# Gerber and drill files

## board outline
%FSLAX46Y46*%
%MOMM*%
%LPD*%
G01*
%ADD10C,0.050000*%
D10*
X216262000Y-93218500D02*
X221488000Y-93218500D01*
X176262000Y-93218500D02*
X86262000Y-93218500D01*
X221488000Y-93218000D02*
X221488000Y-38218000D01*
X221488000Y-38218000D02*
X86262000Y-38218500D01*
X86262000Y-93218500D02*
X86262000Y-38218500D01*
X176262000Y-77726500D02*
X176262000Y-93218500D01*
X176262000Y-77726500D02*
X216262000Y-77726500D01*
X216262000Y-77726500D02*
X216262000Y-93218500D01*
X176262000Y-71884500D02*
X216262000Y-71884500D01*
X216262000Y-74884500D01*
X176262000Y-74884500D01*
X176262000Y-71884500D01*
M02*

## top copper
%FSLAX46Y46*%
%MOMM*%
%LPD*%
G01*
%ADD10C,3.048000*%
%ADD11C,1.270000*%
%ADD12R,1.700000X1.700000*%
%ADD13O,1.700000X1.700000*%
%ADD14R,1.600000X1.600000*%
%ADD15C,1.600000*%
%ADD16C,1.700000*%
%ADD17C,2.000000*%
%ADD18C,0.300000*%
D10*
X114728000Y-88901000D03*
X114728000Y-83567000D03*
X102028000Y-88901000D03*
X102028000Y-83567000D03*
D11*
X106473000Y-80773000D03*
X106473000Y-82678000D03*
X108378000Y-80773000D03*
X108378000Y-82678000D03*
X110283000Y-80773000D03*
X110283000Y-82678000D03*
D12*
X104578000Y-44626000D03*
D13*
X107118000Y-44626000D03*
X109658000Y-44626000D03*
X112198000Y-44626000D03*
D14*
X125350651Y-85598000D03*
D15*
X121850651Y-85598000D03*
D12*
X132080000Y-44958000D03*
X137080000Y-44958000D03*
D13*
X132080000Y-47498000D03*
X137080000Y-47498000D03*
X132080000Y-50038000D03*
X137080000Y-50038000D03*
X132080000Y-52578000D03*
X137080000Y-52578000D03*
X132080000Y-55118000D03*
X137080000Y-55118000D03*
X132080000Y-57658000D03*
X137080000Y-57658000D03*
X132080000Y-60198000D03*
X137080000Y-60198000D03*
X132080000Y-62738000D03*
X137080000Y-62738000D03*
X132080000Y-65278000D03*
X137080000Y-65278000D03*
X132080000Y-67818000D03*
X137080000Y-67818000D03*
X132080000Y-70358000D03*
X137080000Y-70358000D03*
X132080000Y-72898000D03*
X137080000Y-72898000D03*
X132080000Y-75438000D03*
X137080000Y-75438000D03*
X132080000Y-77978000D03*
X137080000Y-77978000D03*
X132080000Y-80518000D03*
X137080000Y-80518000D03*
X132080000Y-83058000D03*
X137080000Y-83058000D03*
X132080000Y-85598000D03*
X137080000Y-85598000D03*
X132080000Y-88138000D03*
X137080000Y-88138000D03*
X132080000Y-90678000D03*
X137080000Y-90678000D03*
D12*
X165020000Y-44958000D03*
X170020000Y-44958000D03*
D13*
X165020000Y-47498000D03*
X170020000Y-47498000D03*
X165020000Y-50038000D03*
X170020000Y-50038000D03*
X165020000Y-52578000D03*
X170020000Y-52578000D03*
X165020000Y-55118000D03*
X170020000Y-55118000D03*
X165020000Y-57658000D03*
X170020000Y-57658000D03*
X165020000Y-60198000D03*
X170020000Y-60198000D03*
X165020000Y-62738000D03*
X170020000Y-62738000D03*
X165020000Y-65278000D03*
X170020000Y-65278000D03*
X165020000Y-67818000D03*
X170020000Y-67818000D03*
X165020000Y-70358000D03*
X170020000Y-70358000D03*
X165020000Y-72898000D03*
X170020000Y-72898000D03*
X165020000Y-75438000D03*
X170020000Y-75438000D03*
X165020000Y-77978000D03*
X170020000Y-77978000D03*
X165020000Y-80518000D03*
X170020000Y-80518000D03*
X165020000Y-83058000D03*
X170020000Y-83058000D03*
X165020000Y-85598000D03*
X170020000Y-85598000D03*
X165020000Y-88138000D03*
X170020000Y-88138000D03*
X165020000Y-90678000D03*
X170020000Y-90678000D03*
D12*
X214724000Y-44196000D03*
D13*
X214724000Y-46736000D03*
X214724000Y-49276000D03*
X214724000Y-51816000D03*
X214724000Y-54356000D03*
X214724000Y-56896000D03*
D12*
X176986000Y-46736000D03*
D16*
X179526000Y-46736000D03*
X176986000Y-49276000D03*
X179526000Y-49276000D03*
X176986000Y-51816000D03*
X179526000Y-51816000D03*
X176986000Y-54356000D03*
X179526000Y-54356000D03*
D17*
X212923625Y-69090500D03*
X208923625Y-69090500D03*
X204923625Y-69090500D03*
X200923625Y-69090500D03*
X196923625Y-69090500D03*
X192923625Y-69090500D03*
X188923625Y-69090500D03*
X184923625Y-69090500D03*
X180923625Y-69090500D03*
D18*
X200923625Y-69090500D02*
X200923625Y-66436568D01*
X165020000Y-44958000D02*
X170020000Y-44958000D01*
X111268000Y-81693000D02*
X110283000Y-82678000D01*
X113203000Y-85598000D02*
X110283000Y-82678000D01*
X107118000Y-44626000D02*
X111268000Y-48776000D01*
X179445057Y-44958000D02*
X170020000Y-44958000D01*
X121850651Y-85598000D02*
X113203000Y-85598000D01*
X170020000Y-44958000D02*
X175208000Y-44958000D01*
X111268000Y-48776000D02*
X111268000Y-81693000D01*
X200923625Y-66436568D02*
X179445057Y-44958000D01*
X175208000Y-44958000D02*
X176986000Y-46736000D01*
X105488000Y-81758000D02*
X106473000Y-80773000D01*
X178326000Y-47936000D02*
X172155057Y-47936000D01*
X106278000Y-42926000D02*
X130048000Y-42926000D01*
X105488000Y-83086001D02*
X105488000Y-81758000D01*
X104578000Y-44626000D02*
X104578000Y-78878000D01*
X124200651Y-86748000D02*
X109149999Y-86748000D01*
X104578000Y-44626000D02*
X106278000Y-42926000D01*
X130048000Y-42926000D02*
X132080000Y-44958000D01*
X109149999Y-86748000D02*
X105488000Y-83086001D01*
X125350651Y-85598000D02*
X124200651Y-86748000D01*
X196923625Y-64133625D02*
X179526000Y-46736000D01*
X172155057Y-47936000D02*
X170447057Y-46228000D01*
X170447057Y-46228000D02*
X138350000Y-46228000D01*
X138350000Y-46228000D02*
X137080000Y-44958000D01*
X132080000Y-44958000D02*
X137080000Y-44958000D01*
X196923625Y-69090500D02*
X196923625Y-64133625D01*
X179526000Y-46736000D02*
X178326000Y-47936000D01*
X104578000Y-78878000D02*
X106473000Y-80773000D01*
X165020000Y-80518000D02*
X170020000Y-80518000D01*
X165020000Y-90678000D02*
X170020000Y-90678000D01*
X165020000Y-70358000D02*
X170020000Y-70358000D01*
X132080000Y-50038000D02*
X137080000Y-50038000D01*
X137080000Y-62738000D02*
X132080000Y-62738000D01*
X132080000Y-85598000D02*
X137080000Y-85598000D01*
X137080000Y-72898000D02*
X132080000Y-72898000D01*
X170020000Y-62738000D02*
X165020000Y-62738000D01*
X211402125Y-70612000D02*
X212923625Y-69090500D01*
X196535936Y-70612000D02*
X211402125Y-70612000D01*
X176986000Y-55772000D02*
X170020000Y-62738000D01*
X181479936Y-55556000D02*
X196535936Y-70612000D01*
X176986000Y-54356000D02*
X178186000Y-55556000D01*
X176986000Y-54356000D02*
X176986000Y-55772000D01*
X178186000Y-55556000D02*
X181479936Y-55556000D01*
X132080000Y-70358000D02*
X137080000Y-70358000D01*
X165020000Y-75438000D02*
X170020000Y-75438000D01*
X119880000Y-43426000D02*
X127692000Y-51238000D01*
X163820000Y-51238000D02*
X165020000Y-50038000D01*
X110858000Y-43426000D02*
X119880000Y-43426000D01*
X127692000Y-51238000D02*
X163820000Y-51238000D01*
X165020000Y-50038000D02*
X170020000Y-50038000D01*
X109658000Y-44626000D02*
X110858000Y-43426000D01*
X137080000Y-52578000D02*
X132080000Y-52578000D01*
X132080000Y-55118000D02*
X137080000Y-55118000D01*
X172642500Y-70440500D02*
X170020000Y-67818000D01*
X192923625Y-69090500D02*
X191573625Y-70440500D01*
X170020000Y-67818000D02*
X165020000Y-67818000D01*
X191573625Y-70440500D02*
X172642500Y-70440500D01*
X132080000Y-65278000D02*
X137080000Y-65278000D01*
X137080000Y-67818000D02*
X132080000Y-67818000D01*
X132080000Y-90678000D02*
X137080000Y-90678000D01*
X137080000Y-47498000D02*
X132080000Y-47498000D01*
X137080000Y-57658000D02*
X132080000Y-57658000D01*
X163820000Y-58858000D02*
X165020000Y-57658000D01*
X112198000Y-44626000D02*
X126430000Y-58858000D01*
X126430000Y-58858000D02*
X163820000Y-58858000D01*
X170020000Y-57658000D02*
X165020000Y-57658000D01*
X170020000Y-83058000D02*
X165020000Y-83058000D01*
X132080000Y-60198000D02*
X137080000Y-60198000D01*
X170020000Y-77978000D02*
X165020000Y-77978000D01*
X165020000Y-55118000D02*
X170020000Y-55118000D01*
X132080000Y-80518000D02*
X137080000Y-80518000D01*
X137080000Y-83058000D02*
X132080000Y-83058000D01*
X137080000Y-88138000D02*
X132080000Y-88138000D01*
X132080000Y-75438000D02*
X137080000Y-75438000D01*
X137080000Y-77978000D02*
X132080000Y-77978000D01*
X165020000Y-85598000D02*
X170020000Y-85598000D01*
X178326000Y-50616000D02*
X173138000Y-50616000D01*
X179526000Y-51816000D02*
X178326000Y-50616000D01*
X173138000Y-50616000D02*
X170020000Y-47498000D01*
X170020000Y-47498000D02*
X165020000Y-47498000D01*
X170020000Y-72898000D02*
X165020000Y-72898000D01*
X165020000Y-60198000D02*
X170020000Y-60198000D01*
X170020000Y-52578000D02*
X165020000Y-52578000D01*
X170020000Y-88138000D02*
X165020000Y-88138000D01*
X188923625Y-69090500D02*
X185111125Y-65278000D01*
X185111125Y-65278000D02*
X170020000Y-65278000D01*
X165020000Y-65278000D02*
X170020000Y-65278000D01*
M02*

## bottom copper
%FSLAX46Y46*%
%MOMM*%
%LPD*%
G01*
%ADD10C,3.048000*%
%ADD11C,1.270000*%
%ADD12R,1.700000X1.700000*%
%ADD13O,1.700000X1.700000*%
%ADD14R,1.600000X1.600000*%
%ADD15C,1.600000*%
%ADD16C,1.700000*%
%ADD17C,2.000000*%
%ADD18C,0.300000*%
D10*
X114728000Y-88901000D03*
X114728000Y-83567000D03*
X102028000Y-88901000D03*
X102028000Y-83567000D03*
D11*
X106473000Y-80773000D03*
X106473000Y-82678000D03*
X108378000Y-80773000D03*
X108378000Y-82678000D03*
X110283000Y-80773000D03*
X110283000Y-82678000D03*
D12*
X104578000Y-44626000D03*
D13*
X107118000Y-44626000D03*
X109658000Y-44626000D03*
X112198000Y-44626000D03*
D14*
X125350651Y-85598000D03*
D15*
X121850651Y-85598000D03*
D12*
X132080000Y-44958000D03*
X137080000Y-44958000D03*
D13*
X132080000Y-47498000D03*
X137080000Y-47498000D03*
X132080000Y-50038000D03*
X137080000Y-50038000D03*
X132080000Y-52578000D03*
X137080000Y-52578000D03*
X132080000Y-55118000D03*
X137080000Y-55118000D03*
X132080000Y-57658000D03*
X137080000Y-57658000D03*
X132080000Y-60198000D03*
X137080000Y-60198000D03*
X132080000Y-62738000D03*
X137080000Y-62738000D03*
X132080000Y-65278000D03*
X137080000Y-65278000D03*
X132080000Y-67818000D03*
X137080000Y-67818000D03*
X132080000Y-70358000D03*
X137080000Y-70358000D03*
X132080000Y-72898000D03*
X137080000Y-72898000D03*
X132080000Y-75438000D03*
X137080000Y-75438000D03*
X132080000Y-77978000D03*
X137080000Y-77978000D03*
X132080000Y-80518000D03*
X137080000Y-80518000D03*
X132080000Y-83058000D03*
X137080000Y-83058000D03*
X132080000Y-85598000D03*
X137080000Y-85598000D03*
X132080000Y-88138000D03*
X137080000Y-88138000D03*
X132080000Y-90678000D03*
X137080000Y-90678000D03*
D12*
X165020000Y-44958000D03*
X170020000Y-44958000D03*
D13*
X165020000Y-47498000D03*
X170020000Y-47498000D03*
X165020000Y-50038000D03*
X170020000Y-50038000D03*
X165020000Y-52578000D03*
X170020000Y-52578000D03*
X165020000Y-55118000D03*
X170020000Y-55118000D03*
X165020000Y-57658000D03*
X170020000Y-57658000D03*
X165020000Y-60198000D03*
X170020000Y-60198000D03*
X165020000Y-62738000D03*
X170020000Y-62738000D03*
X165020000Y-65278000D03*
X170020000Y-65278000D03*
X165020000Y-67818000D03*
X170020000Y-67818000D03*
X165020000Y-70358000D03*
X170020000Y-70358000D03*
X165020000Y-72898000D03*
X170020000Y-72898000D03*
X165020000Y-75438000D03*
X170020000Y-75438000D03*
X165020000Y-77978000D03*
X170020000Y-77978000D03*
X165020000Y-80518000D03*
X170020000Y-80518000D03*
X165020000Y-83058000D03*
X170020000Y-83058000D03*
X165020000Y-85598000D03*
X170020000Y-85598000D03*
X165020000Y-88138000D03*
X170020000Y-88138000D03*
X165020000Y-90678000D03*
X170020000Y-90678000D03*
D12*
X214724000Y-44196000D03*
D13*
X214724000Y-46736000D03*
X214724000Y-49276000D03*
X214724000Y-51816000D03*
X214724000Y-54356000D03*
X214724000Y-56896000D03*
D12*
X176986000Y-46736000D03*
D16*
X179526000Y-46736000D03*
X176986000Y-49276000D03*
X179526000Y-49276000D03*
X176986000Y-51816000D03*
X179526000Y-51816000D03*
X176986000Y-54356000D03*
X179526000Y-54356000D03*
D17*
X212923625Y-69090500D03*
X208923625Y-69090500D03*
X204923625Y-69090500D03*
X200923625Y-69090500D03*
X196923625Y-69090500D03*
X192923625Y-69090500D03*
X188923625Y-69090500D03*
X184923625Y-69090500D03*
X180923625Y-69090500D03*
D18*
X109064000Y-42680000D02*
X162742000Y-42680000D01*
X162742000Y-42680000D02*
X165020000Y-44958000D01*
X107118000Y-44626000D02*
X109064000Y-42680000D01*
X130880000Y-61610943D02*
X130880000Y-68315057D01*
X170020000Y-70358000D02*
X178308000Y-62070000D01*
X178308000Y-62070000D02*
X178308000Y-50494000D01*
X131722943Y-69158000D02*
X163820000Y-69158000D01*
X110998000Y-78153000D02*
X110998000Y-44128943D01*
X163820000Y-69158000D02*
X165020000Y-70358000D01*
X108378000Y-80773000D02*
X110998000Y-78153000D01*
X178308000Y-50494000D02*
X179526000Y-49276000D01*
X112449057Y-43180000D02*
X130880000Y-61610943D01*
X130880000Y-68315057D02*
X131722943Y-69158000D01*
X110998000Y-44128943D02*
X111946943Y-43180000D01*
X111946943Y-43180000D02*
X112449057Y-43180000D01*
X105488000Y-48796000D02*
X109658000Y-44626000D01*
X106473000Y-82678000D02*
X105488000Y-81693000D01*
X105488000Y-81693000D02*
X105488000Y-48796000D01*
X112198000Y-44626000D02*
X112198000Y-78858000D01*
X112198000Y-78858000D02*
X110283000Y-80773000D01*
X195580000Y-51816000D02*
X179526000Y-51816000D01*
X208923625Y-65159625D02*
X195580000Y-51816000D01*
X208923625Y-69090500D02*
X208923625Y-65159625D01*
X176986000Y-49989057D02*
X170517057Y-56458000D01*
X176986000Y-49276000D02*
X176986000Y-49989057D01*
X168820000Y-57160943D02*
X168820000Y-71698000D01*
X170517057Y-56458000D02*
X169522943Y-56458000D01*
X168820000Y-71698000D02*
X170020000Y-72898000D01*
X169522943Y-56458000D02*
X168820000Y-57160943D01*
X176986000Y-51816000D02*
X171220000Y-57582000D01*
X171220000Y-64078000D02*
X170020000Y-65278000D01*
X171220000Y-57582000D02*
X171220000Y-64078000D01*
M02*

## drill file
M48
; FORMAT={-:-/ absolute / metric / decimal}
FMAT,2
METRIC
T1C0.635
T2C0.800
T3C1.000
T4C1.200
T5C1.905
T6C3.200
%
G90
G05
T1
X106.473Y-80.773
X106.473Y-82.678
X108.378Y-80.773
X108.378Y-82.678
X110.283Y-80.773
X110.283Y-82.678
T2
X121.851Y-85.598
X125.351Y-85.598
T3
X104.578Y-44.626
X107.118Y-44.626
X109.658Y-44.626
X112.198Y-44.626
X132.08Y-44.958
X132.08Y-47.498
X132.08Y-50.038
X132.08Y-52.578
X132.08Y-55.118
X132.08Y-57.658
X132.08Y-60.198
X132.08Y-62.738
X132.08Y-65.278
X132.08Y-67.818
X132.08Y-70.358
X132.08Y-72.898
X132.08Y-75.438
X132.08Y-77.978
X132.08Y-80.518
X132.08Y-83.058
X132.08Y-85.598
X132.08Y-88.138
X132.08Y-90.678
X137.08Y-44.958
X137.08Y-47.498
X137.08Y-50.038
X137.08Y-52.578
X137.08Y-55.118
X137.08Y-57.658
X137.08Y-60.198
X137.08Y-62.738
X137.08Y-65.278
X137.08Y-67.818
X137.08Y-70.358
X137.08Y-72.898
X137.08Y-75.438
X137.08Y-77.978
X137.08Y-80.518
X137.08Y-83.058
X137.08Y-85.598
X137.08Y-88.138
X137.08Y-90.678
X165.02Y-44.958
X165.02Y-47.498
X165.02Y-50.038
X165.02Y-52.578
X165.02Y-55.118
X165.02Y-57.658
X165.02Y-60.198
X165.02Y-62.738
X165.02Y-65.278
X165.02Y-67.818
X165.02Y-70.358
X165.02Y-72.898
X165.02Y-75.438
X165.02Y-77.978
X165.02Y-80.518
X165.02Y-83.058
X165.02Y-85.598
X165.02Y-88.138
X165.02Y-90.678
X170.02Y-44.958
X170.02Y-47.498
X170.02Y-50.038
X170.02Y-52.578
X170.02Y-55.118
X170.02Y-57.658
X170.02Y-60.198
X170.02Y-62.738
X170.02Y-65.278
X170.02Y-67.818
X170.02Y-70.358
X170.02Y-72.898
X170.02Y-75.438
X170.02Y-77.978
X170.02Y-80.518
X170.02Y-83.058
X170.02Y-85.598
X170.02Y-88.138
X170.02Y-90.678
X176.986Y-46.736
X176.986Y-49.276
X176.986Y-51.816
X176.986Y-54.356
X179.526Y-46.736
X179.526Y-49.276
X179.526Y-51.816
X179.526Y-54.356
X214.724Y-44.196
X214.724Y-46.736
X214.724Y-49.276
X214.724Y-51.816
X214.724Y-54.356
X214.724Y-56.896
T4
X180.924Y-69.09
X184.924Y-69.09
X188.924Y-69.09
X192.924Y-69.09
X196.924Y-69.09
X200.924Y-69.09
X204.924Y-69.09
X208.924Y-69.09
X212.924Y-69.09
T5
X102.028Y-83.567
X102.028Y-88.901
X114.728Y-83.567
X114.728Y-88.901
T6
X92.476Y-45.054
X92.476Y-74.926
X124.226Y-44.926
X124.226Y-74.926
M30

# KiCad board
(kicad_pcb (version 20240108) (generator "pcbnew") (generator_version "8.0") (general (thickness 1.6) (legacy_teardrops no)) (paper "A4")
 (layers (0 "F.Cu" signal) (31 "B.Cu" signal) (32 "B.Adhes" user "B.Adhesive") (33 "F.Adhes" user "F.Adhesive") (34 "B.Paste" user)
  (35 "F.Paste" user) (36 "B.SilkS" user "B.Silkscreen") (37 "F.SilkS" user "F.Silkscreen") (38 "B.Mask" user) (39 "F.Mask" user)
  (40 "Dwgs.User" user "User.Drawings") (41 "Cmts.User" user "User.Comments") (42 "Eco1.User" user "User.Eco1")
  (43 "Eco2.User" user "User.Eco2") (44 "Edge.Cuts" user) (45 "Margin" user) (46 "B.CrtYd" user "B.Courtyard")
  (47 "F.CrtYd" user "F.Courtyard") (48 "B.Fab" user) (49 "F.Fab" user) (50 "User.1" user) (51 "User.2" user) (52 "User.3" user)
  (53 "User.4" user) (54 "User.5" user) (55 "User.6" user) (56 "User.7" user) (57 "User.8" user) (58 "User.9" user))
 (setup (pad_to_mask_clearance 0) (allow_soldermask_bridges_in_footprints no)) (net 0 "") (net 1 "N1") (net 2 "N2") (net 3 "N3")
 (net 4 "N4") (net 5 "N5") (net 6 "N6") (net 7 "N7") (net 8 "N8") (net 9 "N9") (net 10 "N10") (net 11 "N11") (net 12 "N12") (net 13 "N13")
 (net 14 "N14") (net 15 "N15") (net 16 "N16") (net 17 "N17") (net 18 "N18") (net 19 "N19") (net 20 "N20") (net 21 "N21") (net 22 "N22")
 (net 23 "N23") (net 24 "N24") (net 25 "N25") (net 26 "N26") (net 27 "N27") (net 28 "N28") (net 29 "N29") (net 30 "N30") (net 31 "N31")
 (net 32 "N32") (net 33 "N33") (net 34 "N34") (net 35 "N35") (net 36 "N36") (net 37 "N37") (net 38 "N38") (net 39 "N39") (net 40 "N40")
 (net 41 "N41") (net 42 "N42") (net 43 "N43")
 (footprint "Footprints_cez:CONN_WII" (layer "F.Cu") (at 108.378 86.361 180)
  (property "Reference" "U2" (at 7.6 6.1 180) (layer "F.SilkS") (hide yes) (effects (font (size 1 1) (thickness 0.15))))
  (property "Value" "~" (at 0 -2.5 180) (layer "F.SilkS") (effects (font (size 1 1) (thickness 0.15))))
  (pad "" thru_hole circle (at -6.35 -2.54 180) (size 3.048 3.048) (drill 1.905) (layers "*.Cu" "*.Mask") (remove_unused_layers no))
  (pad "" thru_hole circle (at -6.35 2.794 180) (size 3.048 3.048) (drill 1.905) (layers "*.Cu" "*.Mask") (remove_unused_layers no))
  (pad "" thru_hole circle (at 6.35 -2.54 180) (size 3.048 3.048) (drill 1.905) (layers "*.Cu" "*.Mask") (remove_unused_layers no))
  (pad "" thru_hole circle (at 6.35 2.794 180) (size 3.048 3.048) (drill 1.905) (layers "*.Cu" "*.Mask") (remove_unused_layers no))
  (pad "1" thru_hole circle (at 1.905 5.588 180) (size 1.27 1.27) (drill 0.635) (layers "*.Cu" "*.Mask") (remove_unused_layers no)
   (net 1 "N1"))
  (pad "2" thru_hole circle (at 1.905 3.683 180) (size 1.27 1.27) (drill 0.635) (layers "*.Cu" "*.Mask") (remove_unused_layers no)
   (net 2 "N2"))
  (pad "3" thru_hole circle (at 0 5.588 180) (size 1.27 1.27) (drill 0.635) (layers "*.Cu" "*.Mask") (remove_unused_layers no) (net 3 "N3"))
  (pad "4" thru_hole circle (at 0 3.683 180) (size 1.27 1.27) (drill 0.635) (layers "*.Cu" "*.Mask") (remove_unused_layers no) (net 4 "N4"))
  (pad "5" thru_hole circle (at -1.905 5.588 180) (size 1.27 1.27) (drill 0.635) (layers "*.Cu" "*.Mask") (remove_unused_layers no)
   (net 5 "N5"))
  (pad "6" thru_hole circle (at -1.905 3.683 180) (size 1.27 1.27) (drill 0.635) (layers "*.Cu" "*.Mask") (remove_unused_layers no)
   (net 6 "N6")))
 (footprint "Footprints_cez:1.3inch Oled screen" (layer "F.Cu") (at 108.478 36.926)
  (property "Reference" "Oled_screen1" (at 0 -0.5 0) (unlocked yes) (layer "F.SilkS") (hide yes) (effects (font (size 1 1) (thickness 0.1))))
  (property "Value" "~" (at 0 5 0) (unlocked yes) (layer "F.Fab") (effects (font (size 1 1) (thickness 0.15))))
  (pad "" np_thru_hole circle (at -16.002 8.128) (size 3.2 3.2) (drill 3.2) (layers "*.Cu" "*.Mask"))
  (pad "" np_thru_hole circle (at -16.002 38) (size 3.2 3.2) (drill 3.2) (layers "*.Cu" "*.Mask"))
  (pad "" np_thru_hole circle (at 15.748 8) (size 3.2 3.2) (drill 3.2) (layers "*.Cu" "*.Mask"))
  (pad "" np_thru_hole circle (at 15.748 38) (size 3.2 3.2) (drill 3.2) (layers "*.Cu" "*.Mask"))
  (pad "1" thru_hole rect (at -3.9 7.7 90) (size 1.7 1.7) (drill 1) (layers "*.Cu" "*.Mask") (remove_unused_layers no) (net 1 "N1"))
  (pad "2" thru_hole oval (at -1.36 7.7 90) (size 1.7 1.7) (drill 1) (layers "*.Cu" "*.Mask") (remove_unused_layers no) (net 6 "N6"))
  (pad "3" thru_hole oval (at 1.18 7.7 90) (size 1.7 1.7) (drill 1) (layers "*.Cu" "*.Mask") (remove_unused_layers no) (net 2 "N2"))
  (pad "4" thru_hole oval (at 3.72 7.7 90) (size 1.7 1.7) (drill 1) (layers "*.Cu" "*.Mask") (remove_unused_layers no) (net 5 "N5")))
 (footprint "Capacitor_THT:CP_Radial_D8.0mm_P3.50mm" (layer "F.Cu") (at 125.350651 85.598 180)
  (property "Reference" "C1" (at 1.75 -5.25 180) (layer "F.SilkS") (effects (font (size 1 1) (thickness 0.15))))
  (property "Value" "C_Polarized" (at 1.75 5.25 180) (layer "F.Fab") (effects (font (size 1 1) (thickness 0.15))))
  (pad "1" thru_hole rect (at 0 0 180) (size 1.6 1.6) (drill 0.8) (layers "*.Cu" "*.Mask") (remove_unused_layers no) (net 1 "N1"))
  (pad "2" thru_hole circle (at 3.5 0 180) (size 1.6 1.6) (drill 0.8) (layers "*.Cu" "*.Mask") (remove_unused_layers no) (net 6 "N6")))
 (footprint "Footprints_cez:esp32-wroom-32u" (layer "F.Cu") (at 149.78 57.14)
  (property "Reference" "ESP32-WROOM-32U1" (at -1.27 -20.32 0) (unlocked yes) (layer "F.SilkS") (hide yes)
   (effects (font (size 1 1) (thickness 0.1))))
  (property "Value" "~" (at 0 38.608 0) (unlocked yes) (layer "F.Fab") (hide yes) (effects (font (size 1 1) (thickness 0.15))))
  (pad "1" thru_hole rect (at -17.7 -12.182) (size 1.7 1.7) (drill 1) (layers "*.Cu" "*.Mask") (remove_unused_layers no) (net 1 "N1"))
  (pad "1" thru_hole rect (at -12.7 -12.182) (size 1.7 1.7) (drill 1) (layers "*.Cu" "*.Mask") (remove_unused_layers no) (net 1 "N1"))
  (pad "2" thru_hole oval (at -17.7 -9.642) (size 1.7 1.7) (drill 1) (layers "*.Cu" "*.Mask") (remove_unused_layers no) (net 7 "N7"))
  (pad "2" thru_hole oval (at -12.7 -9.642) (size 1.7 1.7) (drill 1) (layers "*.Cu" "*.Mask") (remove_unused_layers no) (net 7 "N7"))
  (pad "3" thru_hole oval (at -17.7 -7.102) (size 1.7 1.7) (drill 1) (layers "*.Cu" "*.Mask") (remove_unused_layers no) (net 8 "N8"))
  (pad "3" thru_hole oval (at -12.7 -7.102) (size 1.7 1.7) (drill 1) (layers "*.Cu" "*.Mask") (remove_unused_layers no) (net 8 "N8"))
  (pad "4" thru_hole oval (at -17.7 -4.562) (size 1.7 1.7) (drill 1) (layers "*.Cu" "*.Mask") (remove_unused_layers no) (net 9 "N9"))
  (pad "4" thru_hole oval (at -12.7 -4.562) (size 1.7 1.7) (drill 1) (layers "*.Cu" "*.Mask") (remove_unused_layers no) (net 9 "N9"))
  (pad "5" thru_hole oval (at -17.7 -2.022) (size 1.7 1.7) (drill 1) (layers "*.Cu" "*.Mask") (remove_unused_layers no) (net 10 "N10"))
  (pad "5" thru_hole oval (at -12.7 -2.022) (size 1.7 1.7) (drill 1) (layers "*.Cu" "*.Mask") (remove_unused_layers no) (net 10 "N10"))
  (pad "6" thru_hole oval (at -17.7 0.518) (size 1.7 1.7) (drill 1) (layers "*.Cu" "*.Mask") (remove_unused_layers no) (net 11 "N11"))
  (pad "6" thru_hole oval (at -12.7 0.518) (size 1.7 1.7) (drill 1) (layers "*.Cu" "*.Mask") (remove_unused_layers no) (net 11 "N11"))
  (pad "7" thru_hole oval (at -17.7 3.058) (size 1.7 1.7) (drill 1) (layers "*.Cu" "*.Mask") (remove_unused_layers no) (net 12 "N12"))
  (pad "7" thru_hole oval (at -12.7 3.058) (size 1.7 1.7) (drill 1) (layers "*.Cu" "*.Mask") (remove_unused_layers no) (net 12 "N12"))
  (pad "8" thru_hole oval (at -17.7 5.598) (size 1.7 1.7) (drill 1) (layers "*.Cu" "*.Mask") (remove_unused_layers no) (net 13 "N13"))
  (pad "8" thru_hole oval (at -12.7 5.598) (size 1.7 1.7) (drill 1) (layers "*.Cu" "*.Mask") (remove_unused_layers no) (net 13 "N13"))
  (pad "9" thru_hole oval (at -17.7 8.138) (size 1.7 1.7) (drill 1) (layers "*.Cu" "*.Mask") (remove_unused_layers no) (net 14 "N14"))
  (pad "9" thru_hole oval (at -12.7 8.138) (size 1.7 1.7) (drill 1) (layers "*.Cu" "*.Mask") (remove_unused_layers no) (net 14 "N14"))
  (pad "10" thru_hole oval (at -17.7 10.678) (size 1.7 1.7) (drill 1) (layers "*.Cu" "*.Mask") (remove_unused_layers no) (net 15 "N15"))
  (pad "10" thru_hole oval (at -12.7 10.678) (size 1.7 1.7) (drill 1) (layers "*.Cu" "*.Mask") (remove_unused_layers no) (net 15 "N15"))
  (pad "11" thru_hole oval (at -17.7 13.218) (size 1.7 1.7) (drill 1) (layers "*.Cu" "*.Mask") (remove_unused_layers no) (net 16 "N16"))
  (pad "11" thru_hole oval (at -12.7 13.218) (size 1.7 1.7) (drill 1) (layers "*.Cu" "*.Mask") (remove_unused_layers no) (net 16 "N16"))
  (pad "12" thru_hole oval (at -17.7 15.758) (size 1.7 1.7) (drill 1) (layers "*.Cu" "*.Mask") (remove_unused_layers no) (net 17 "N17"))
  (pad "12" thru_hole oval (at -12.7 15.758) (size 1.7 1.7) (drill 1) (layers "*.Cu" "*.Mask") (remove_unused_layers no) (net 17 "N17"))
  (pad "13" thru_hole oval (at -17.7 18.298) (size 1.7 1.7) (drill 1) (layers "*.Cu" "*.Mask") (remove_unused_layers no) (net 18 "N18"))
  (pad "13" thru_hole oval (at -12.7 18.298) (size 1.7 1.7) (drill 1) (layers "*.Cu" "*.Mask") (remove_unused_layers no) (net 18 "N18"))
  (pad "14" thru_hole oval (at -17.7 20.838) (size 1.7 1.7) (drill 1) (layers "*.Cu" "*.Mask") (remove_unused_layers no) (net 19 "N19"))
  (pad "14" thru_hole oval (at -12.7 20.838) (size 1.7 1.7) (drill 1) (layers "*.Cu" "*.Mask") (remove_unused_layers no) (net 19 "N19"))
  (pad "15" thru_hole oval (at -17.7 23.378) (size 1.7 1.7) (drill 1) (layers "*.Cu" "*.Mask") (remove_unused_layers no) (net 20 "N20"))
  (pad "15" thru_hole oval (at -12.7 23.378) (size 1.7 1.7) (drill 1) (layers "*.Cu" "*.Mask") (remove_unused_layers no) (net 20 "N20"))
  (pad "16" thru_hole oval (at -17.7 25.918) (size 1.7 1.7) (drill 1) (layers "*.Cu" "*.Mask") (remove_unused_layers no) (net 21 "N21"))
  (pad "16" thru_hole oval (at -12.7 25.918) (size 1.7 1.7) (drill 1) (layers "*.Cu" "*.Mask") (remove_unused_layers no) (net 21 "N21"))
  (pad "17" thru_hole oval (at -17.7 28.458) (size 1.7 1.7) (drill 1) (layers "*.Cu" "*.Mask") (remove_unused_layers no) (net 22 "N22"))
  (pad "17" thru_hole oval (at -12.7 28.458) (size 1.7 1.7) (drill 1) (layers "*.Cu" "*.Mask") (remove_unused_layers no) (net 22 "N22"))
  (pad "18" thru_hole oval (at -17.7 30.998) (size 1.7 1.7) (drill 1) (layers "*.Cu" "*.Mask") (remove_unused_layers no) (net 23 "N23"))
  (pad "18" thru_hole oval (at -12.7 30.998) (size 1.7 1.7) (drill 1) (layers "*.Cu" "*.Mask") (remove_unused_layers no) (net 23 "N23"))
  (pad "19" thru_hole oval (at -17.7 33.538) (size 1.7 1.7) (drill 1) (layers "*.Cu" "*.Mask") (remove_unused_layers no) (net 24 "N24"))
  (pad "19" thru_hole oval (at -12.7 33.538) (size 1.7 1.7) (drill 1) (layers "*.Cu" "*.Mask") (remove_unused_layers no) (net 24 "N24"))
  (pad "20" thru_hole rect (at 15.24 -12.182) (size 1.7 1.7) (drill 1) (layers "*.Cu" "*.Mask") (remove_unused_layers no) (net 6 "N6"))
  (pad "20" thru_hole rect (at 20.24 -12.182) (size 1.7 1.7) (drill 1) (layers "*.Cu" "*.Mask") (remove_unused_layers no) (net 6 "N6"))
  (pad "21" thru_hole oval (at 15.24 -9.642) (size 1.7 1.7) (drill 1) (layers "*.Cu" "*.Mask") (remove_unused_layers no) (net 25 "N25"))
  (pad "21" thru_hole oval (at 20.24 -9.642) (size 1.7 1.7) (drill 1) (layers "*.Cu" "*.Mask") (remove_unused_layers no) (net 25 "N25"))
  (pad "22" thru_hole oval (at 15.24 -7.102) (size 1.7 1.7) (drill 1) (layers "*.Cu" "*.Mask") (remove_unused_layers no) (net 2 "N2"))
  (pad "22" thru_hole oval (at 20.24 -7.102) (size 1.7 1.7) (drill 1) (layers "*.Cu" "*.Mask") (remove_unused_layers no) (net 2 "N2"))
  (pad "23" thru_hole oval (at 15.24 -4.562) (size 1.7 1.7) (drill 1) (layers "*.Cu" "*.Mask") (remove_unused_layers no) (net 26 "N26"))
  (pad "23" thru_hole oval (at 20.24 -4.562) (size 1.7 1.7) (drill 1) (layers "*.Cu" "*.Mask") (remove_unused_layers no) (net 26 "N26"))
  (pad "24" thru_hole oval (at 15.24 -2.022) (size 1.7 1.7) (drill 1) (layers "*.Cu" "*.Mask") (remove_unused_layers no) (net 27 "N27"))
  (pad "24" thru_hole oval (at 20.24 -2.022) (size 1.7 1.7) (drill 1) (layers "*.Cu" "*.Mask") (remove_unused_layers no) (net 27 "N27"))
  (pad "25" thru_hole oval (at 15.24 0.518) (size 1.7 1.7) (drill 1) (layers "*.Cu" "*.Mask") (remove_unused_layers no) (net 5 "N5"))
  (pad "25" thru_hole oval (at 20.24 0.518) (size 1.7 1.7) (drill 1) (layers "*.Cu" "*.Mask") (remove_unused_layers no) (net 5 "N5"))
  (pad "26" thru_hole oval (at 15.24 3.058) (size 1.7 1.7) (drill 1) (layers "*.Cu" "*.Mask") (remove_unused_layers no) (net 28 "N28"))
  (pad "26" thru_hole oval (at 20.24 3.058) (size 1.7 1.7) (drill 1) (layers "*.Cu" "*.Mask") (remove_unused_layers no) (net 28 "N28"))
  (pad "27" thru_hole oval (at 15.24 5.598) (size 1.7 1.7) (drill 1) (layers "*.Cu" "*.Mask") (remove_unused_layers no) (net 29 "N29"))
  (pad "27" thru_hole oval (at 20.24 5.598) (size 1.7 1.7) (drill 1) (layers "*.Cu" "*.Mask") (remove_unused_layers no) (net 29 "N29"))
  (pad "28" thru_hole oval (at 15.24 8.138) (size 1.7 1.7) (drill 1) (layers "*.Cu" "*.Mask") (remove_unused_layers no) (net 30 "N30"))
  (pad "28" thru_hole oval (at 20.24 8.138) (size 1.7 1.7) (drill 1) (layers "*.Cu" "*.Mask") (remove_unused_layers no) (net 30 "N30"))
  (pad "29" thru_hole oval (at 15.24 10.678) (size 1.7 1.7) (drill 1) (layers "*.Cu" "*.Mask") (remove_unused_layers no) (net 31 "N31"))
  (pad "29" thru_hole oval (at 20.24 10.678) (size 1.7 1.7) (drill 1) (layers "*.Cu" "*.Mask") (remove_unused_layers no) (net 31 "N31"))
  (pad "30" thru_hole oval (at 15.24 13.218) (size 1.7 1.7) (drill 1) (layers "*.Cu" "*.Mask") (remove_unused_layers no) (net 3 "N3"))
  (pad "30" thru_hole oval (at 20.24 13.218) (size 1.7 1.7) (drill 1) (layers "*.Cu" "*.Mask") (remove_unused_layers no) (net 3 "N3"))
  (pad "31" thru_hole oval (at 15.24 15.758) (size 1.7 1.7) (drill 1) (layers "*.Cu" "*.Mask") (remove_unused_layers no) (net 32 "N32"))
  (pad "31" thru_hole oval (at 20.24 15.758) (size 1.7 1.7) (drill 1) (layers "*.Cu" "*.Mask") (remove_unused_layers no) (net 32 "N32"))
  (pad "32" thru_hole oval (at 15.24 18.298) (size 1.7 1.7) (drill 1) (layers "*.Cu" "*.Mask") (remove_unused_layers no) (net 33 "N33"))
  (pad "32" thru_hole oval (at 20.24 18.298) (size 1.7 1.7) (drill 1) (layers "*.Cu" "*.Mask") (remove_unused_layers no) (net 33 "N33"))
  (pad "33" thru_hole oval (at 15.24 20.838) (size 1.7 1.7) (drill 1) (layers "*.Cu" "*.Mask") (remove_unused_layers no) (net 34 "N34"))
  (pad "33" thru_hole oval (at 20.24 20.838) (size 1.7 1.7) (drill 1) (layers "*.Cu" "*.Mask") (remove_unused_layers no) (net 34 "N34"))
  (pad "34" thru_hole oval (at 15.24 23.378) (size 1.7 1.7) (drill 1) (layers "*.Cu" "*.Mask") (remove_unused_layers no) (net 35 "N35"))
  (pad "34" thru_hole oval (at 20.24 23.378) (size 1.7 1.7) (drill 1) (layers "*.Cu" "*.Mask") (remove_unused_layers no) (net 35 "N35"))
  (pad "35" thru_hole oval (at 15.24 25.918) (size 1.7 1.7) (drill 1) (layers "*.Cu" "*.Mask") (remove_unused_layers no) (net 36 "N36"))
  (pad "35" thru_hole oval (at 20.24 25.918) (size 1.7 1.7) (drill 1) (layers "*.Cu" "*.Mask") (remove_unused_layers no) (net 36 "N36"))
  (pad "36" thru_hole oval (at 15.24 28.458) (size 1.7 1.7) (drill 1) (layers "*.Cu" "*.Mask") (remove_unused_layers no) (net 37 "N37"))
  (pad "36" thru_hole oval (at 20.24 28.458) (size 1.7 1.7) (drill 1) (layers "*.Cu" "*.Mask") (remove_unused_layers no) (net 37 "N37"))
  (pad "37" thru_hole oval (at 15.24 30.998) (size 1.7 1.7) (drill 1) (layers "*.Cu" "*.Mask") (remove_unused_layers no) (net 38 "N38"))
  (pad "37" thru_hole oval (at 20.24 30.998) (size 1.7 1.7) (drill 1) (layers "*.Cu" "*.Mask") (remove_unused_layers no) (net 38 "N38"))
  (pad "38" thru_hole oval (at 15.24 33.538) (size 1.7 1.7) (drill 1) (layers "*.Cu" "*.Mask") (remove_unused_layers no) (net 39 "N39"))
  (pad "38" thru_hole oval (at 20.24 33.538) (size 1.7 1.7) (drill 1) (layers "*.Cu" "*.Mask") (remove_unused_layers no) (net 39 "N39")))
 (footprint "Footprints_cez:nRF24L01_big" (layer "F.Cu") (at 176.986 46.736)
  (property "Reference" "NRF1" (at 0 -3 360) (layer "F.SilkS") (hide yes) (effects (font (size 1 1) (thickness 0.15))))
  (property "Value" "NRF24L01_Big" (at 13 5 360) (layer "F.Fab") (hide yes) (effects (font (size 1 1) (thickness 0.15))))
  (pad "" thru_hole rect (at 37.738 -2.54) (size 1.7 1.7) (drill 1) (layers "*.Cu" "*.Mask") (remove_unused_layers no))
  (pad "" thru_hole oval (at 37.738 0) (size 1.7 1.7) (drill 1) (layers "*.Cu" "*.Mask") (remove_unused_layers no))
  (pad "" thru_hole oval (at 37.738 2.54) (size 1.7 1.7) (drill 1) (layers "*.Cu" "*.Mask") (remove_unused_layers no))
  (pad "" thru_hole oval (at 37.738 5.08) (size 1.7 1.7) (drill 1) (layers "*.Cu" "*.Mask") (remove_unused_layers no))
  (pad "" thru_hole oval (at 37.738 7.62) (size 1.7 1.7) (drill 1) (layers "*.Cu" "*.Mask") (remove_unused_layers no))
  (pad "" thru_hole oval (at 37.738 10.16) (size 1.7 1.7) (drill 1) (layers "*.Cu" "*.Mask") (remove_unused_layers no))
  (pad "1" thru_hole rect (at 0 0) (size 1.7 1.7) (drill 1) (layers "*.Cu" "*.Mask") (remove_unused_layers no) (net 6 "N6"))
  (pad "2" thru_hole circle (at 2.54 0) (size 1.7 1.7) (drill 1) (layers "*.Cu" "*.Mask") (remove_unused_layers no) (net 1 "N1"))
  (pad "3" thru_hole circle (at 0 2.54) (size 1.7 1.7) (drill 1) (layers "*.Cu" "*.Mask") (remove_unused_layers no) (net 32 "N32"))
  (pad "4" thru_hole circle (at 2.54 2.54) (size 1.7 1.7) (drill 1) (layers "*.Cu" "*.Mask") (remove_unused_layers no) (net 3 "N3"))
  (pad "5" thru_hole circle (at 0 5.08) (size 1.7 1.7) (drill 1) (layers "*.Cu" "*.Mask") (remove_unused_layers no) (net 30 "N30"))
  (pad "6" thru_hole circle (at 2.54 5.08) (size 1.7 1.7) (drill 1) (layers "*.Cu" "*.Mask") (remove_unused_layers no) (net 25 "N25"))
  (pad "7" thru_hole circle (at 0 7.62) (size 1.7 1.7) (drill 1) (layers "*.Cu" "*.Mask") (remove_unused_layers no) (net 29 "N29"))
  (pad "8" thru_hole circle (at 2.54 7.62) (size 1.7 1.7) (drill 1) (layers "*.Cu" "*.Mask") (remove_unused_layers no) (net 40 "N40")))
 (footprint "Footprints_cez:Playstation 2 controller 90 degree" (layer "F.Cu") (at 193.606625 64.6465 90)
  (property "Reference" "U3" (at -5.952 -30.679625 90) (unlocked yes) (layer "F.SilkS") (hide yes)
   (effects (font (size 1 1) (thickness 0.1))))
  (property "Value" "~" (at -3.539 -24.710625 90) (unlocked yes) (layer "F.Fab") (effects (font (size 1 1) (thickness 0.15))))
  (fp_line (start -13.08 -17.344625) (end -28.572 -17.344625) (stroke (width 0.05) (type default)) (layer "Edge.Cuts"))
  (fp_line (start -13.08 -17.344625) (end -13.08 22.655375) (stroke (width 0.05) (type default)) (layer "Edge.Cuts"))
  (fp_line (start -13.08 22.655375) (end -28.572 22.655375) (stroke (width 0.05) (type default)) (layer "Edge.Cuts"))
  (fp_rect (start -10.238 -17.344625) (end -7.238 22.655375) (stroke (width 0.05) (type default)) (fill none) (layer "Edge.Cuts"))
  (pad "1" thru_hole circle (at -4.444 19.317 90) (size 2 2) (drill 1.2) (layers "*.Cu" "*.Mask") (remove_unused_layers no) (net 29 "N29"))
  (pad "2" thru_hole circle (at -4.444 15.317 90) (size 2 2) (drill 1.2) (layers "*.Cu" "*.Mask") (remove_unused_layers no) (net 25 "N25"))
  (pad "3" thru_hole circle (at -4.444 11.317 90) (size 2 2) (drill 1.2) (layers "*.Cu" "*.Mask") (remove_unused_layers no) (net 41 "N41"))
  (pad "4" thru_hole circle (at -4.444 7.317 90) (size 2 2) (drill 1.2) (layers "*.Cu" "*.Mask") (remove_unused_layers no) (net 6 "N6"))
  (pad "5" thru_hole circle (at -4.444 3.317 90) (size 2 2) (drill 1.2) (layers "*.Cu" "*.Mask") (remove_unused_layers no) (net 1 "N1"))
  (pad "6" thru_hole circle (at -4.444 -0.683 90) (size 2 2) (drill 1.2) (layers "*.Cu" "*.Mask") (remove_unused_layers no) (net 31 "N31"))
  (pad "7" thru_hole circle (at -4.444 -4.683 90) (size 2 2) (drill 1.2) (layers "*.Cu" "*.Mask") (remove_unused_layers no) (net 30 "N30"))
  (pad "8" thru_hole circle (at -4.444 -8.683 90) (size 2 2) (drill 1.2) (layers "*.Cu" "*.Mask") (remove_unused_layers no) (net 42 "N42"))
  (pad "9" thru_hole circle (at -4.444 -12.683 90) (size 2 2) (drill 1.2) (layers "*.Cu" "*.Mask") (remove_unused_layers no) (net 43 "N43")))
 (gr_line (start 216.262 93.2185) (end 221.488 93.2185) (stroke (width 0.05) (type default)) (layer "Edge.Cuts"))
 (gr_line (start 176.262 93.2185) (end 86.262 93.2185) (stroke (width 0.05) (type default)) (layer "Edge.Cuts"))
 (gr_line (start 221.488 93.218) (end 221.488 38.218) (stroke (width 0.05) (type default)) (layer "Edge.Cuts"))
 (gr_line (start 221.488 38.218) (end 86.262 38.2185) (stroke (width 0.05) (type default)) (layer "Edge.Cuts"))
 (gr_line (start 86.262 93.2185) (end 86.262 38.2185) (stroke (width 0.05) (type default)) (layer "Edge.Cuts"))
 (segment (start 200.923625 69.0905) (end 200.923625 66.436568) (width 0.3) (layer "F.Cu") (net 6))
 (segment (start 165.02 44.958) (end 170.02 44.958) (width 0.3) (layer "F.Cu") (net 6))
 (segment (start 111.268 81.693) (end 110.283 82.678) (width 0.3) (layer "F.Cu") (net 6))
 (segment (start 113.203 85.598) (end 110.283 82.678) (width 0.3) (layer "F.Cu") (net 6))
 (segment (start 107.118 44.626) (end 111.268 48.776) (width 0.3) (layer "F.Cu") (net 6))
 (segment (start 179.445057 44.958) (end 170.02 44.958) (width 0.3) (layer "F.Cu") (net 6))
 (segment (start 121.850651 85.598) (end 113.203 85.598) (width 0.3) (layer "F.Cu") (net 6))
 (segment (start 170.02 44.958) (end 175.208 44.958) (width 0.3) (layer "F.Cu") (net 6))
 (segment (start 111.268 48.776) (end 111.268 81.693) (width 0.3) (layer "F.Cu") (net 6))
 (segment (start 200.923625 66.436568) (end 179.445057 44.958) (width 0.3) (layer "F.Cu") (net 6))
 (segment (start 175.208 44.958) (end 176.986 46.736) (width 0.3) (layer "F.Cu") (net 6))
 (segment (start 109.064 42.68) (end 162.742 42.68) (width 0.3) (layer "B.Cu") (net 6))
 (segment (start 162.742 42.68) (end 165.02 44.958) (width 0.3) (layer "B.Cu") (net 6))
 (segment (start 107.118 44.626) (end 109.064 42.68) (width 0.3) (layer "B.Cu") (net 6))
 (segment (start 105.488 81.758) (end 106.473 80.773) (width 0.3) (layer "F.Cu") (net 1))
 (segment (start 178.326 47.936) (end 172.155057 47.936) (width 0.3) (layer "F.Cu") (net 1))
 (segment (start 106.278 42.926) (end 130.048 42.926) (width 0.3) (layer "F.Cu") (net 1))
 (segment (start 105.488 83.086001) (end 105.488 81.758) (width 0.3) (layer "F.Cu") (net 1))
 (segment (start 104.578 44.626) (end 104.578 78.878) (width 0.3) (layer "F.Cu") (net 1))
 (segment (start 124.200651 86.748) (end 109.149999 86.748) (width 0.3) (layer "F.Cu") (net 1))
 (segment (start 104.578 44.626) (end 106.278 42.926) (width 0.3) (layer "F.Cu") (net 1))
 (segment (start 130.048 42.926) (end 132.08 44.958) (width 0.3) (layer "F.Cu") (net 1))
 (segment (start 109.149999 86.748) (end 105.488 83.086001) (width 0.3) (layer "F.Cu") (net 1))
 (segment (start 125.350651 85.598) (end 124.200651 86.748) (width 0.3) (layer "F.Cu") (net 1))
 (segment (start 196.923625 64.133625) (end 179.526 46.736) (width 0.3) (layer "F.Cu") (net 1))
 (segment (start 172.155057 47.936) (end 170.447057 46.228) (width 0.3) (layer "F.Cu") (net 1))
 (segment (start 170.447057 46.228) (end 138.35 46.228) (width 0.3) (layer "F.Cu") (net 1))
 (segment (start 138.35 46.228) (end 137.08 44.958) (width 0.3) (layer "F.Cu") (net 1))
 (segment (start 132.08 44.958) (end 137.08 44.958) (width 0.3) (layer "F.Cu") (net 1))
 (segment (start 196.923625 69.0905) (end 196.923625 64.133625) (width 0.3) (layer "F.Cu") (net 1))
 (segment (start 179.526 46.736) (end 178.326 47.936) (width 0.3) (layer "F.Cu") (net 1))
 (segment (start 104.578 78.878) (end 106.473 80.773) (width 0.3) (layer "F.Cu") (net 1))
 (segment (start 165.02 80.518) (end 170.02 80.518) (width 0.3) (layer "F.Cu") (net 35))
 (segment (start 165.02 90.678) (end 170.02 90.678) (width 0.3) (layer "F.Cu") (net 39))
 (segment (start 165.02 70.358) (end 170.02 70.358) (width 0.3) (layer "F.Cu") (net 3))
 (segment (start 130.88 61.610943) (end 130.88 68.315057) (width 0.3) (layer "B.Cu") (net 3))
 (segment (start 170.02 70.358) (end 178.308 62.07) (width 0.3) (layer "B.Cu") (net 3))
 (segment (start 178.308 62.07) (end 178.308 50.494) (width 0.3) (layer "B.Cu") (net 3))
 (segment (start 131.722943 69.158) (end 163.82 69.158) (width 0.3) (layer "B.Cu") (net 3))
 (segment (start 110.998 78.153) (end 110.998 44.128943) (width 0.3) (layer "B.Cu") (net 3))
 (segment (start 163.82 69.158) (end 165.02 70.358) (width 0.3) (layer "B.Cu") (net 3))
 (segment (start 108.378 80.773) (end 110.998 78.153) (width 0.3) (layer "B.Cu") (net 3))
 (segment (start 178.308 50.494) (end 179.526 49.276) (width 0.3) (layer "B.Cu") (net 3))
 (segment (start 112.449057 43.18) (end 130.88 61.610943) (width 0.3) (layer "B.Cu") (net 3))
 (segment (start 130.88 68.315057) (end 131.722943 69.158) (width 0.3) (layer "B.Cu") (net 3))
 (segment (start 110.998 44.128943) (end 111.946943 43.18) (width 0.3) (layer "B.Cu") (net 3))
 (segment (start 111.946943 43.18) (end 112.449057 43.18) (width 0.3) (layer "B.Cu") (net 3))
 (segment (start 132.08 50.038) (end 137.08 50.038) (width 0.3) (layer "F.Cu") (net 8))
 (segment (start 137.08 62.738) (end 132.08 62.738) (width 0.3) (layer "F.Cu") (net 13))
 (segment (start 132.08 85.598) (end 137.08 85.598) (width 0.3) (layer "F.Cu") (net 22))
 (segment (start 137.08 72.898) (end 132.08 72.898) (width 0.3) (layer "F.Cu") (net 17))
 (segment (start 170.02 62.738) (end 165.02 62.738) (width 0.3) (layer "F.Cu") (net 29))
 (segment (start 211.402125 70.612) (end 212.923625 69.0905) (width 0.3) (layer "F.Cu") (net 29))
 (segment (start 196.535936 70.612) (end 211.402125 70.612) (width 0.3) (layer "F.Cu") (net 29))
 (segment (start 176.986 55.772) (end 170.02 62.738) (width 0.3) (layer "F.Cu") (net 29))
 (segment (start 181.479936 55.556) (end 196.535936 70.612) (width 0.3) (layer "F.Cu") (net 29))
 (segment (start 176.986 54.356) (end 178.186 55.556) (width 0.3) (layer "F.Cu") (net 29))
 (segment (start 176.986 54.356) (end 176.986 55.772) (width 0.3) (layer "F.Cu") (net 29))
 (segment (start 178.186 55.556) (end 181.479936 55.556) (width 0.3) (layer "F.Cu") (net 29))
 (segment (start 132.08 70.358) (end 137.08 70.358) (width 0.3) (layer "F.Cu") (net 16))
 (segment (start 165.02 75.438) (end 170.02 75.438) (width 0.3) (layer "F.Cu") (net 33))
 (segment (start 119.88 43.426) (end 127.692 51.238) (width 0.3) (layer "F.Cu") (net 2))
 (segment (start 163.82 51.238) (end 165.02 50.038) (width 0.3) (layer "F.Cu") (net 2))
 (segment (start 110.858 43.426) (end 119.88 43.426) (width 0.3) (layer "F.Cu") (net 2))
 (segment (start 127.692 51.238) (end 163.82 51.238) (width 0.3) (layer "F.Cu") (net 2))
 (segment (start 165.02 50.038) (end 170.02 50.038) (width 0.3) (layer "F.Cu") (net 2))
 (segment (start 109.658 44.626) (end 110.858 43.426) (width 0.3) (layer "F.Cu") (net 2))
 (segment (start 105.488 48.796) (end 109.658 44.626) (width 0.3) (layer "B.Cu") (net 2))
 (segment (start 106.473 82.678) (end 105.488 81.693) (width 0.3) (layer "B.Cu") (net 2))
 (segment (start 105.488 81.693) (end 105.488 48.796) (width 0.3) (layer "B.Cu") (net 2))
 (segment (start 137.08 52.578) (end 132.08 52.578) (width 0.3) (layer "F.Cu") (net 9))
 (segment (start 132.08 55.118) (end 137.08 55.118) (width 0.3) (layer "F.Cu") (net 10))
 (segment (start 172.6425 70.4405) (end 170.02 67.818) (width 0.3) (layer "F.Cu") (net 31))
 (segment (start 192.923625 69.0905) (end 191.573625 70.4405) (width 0.3) (layer "F.Cu") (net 31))
 (segment (start 170.02 67.818) (end 165.02 67.818) (width 0.3) (layer "F.Cu") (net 31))
 (segment (start 191.573625 70.4405) (end 172.6425 70.4405) (width 0.3) (layer "F.Cu") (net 31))
 (segment (start 132.08 65.278) (end 137.08 65.278) (width 0.3) (layer "F.Cu") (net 14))
 (segment (start 137.08 67.818) (end 132.08 67.818) (width 0.3) (layer "F.Cu") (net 15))
 (segment (start 132.08 90.678) (end 137.08 90.678) (width 0.3) (layer "F.Cu") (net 24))
 (segment (start 137.08 47.498) (end 132.08 47.498) (width 0.3) (layer "F.Cu") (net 7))
 (segment (start 137.08 57.658) (end 132.08 57.658) (width 0.3) (layer "F.Cu") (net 11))
 (segment (start 163.82 58.858) (end 165.02 57.658) (width 0.3) (layer "F.Cu") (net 5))
 (segment (start 112.198 44.626) (end 126.43 58.858) (width 0.3) (layer "F.Cu") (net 5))
 (segment (start 126.43 58.858) (end 163.82 58.858) (width 0.3) (layer "F.Cu") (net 5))
 (segment (start 170.02 57.658) (end 165.02 57.658) (width 0.3) (layer "F.Cu") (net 5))
 (segment (start 112.198 44.626) (end 112.198 78.858) (width 0.3) (layer "B.Cu") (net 5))
 (segment (start 112.198 78.858) (end 110.283 80.773) (width 0.3) (layer "B.Cu") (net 5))
 (segment (start 170.02 83.058) (end 165.02 83.058) (width 0.3) (layer "F.Cu") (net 36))
 (segment (start 132.08 60.198) (end 137.08 60.198) (width 0.3) (layer "F.Cu") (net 12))
 (segment (start 170.02 77.978) (end 165.02 77.978) (width 0.3) (layer "F.Cu") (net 34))
 (segment (start 165.02 55.118) (end 170.02 55.118) (width 0.3) (layer "F.Cu") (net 27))
 (segment (start 132.08 80.518) (end 137.08 80.518) (width 0.3) (layer "F.Cu") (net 20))
 (segment (start 137.08 83.058) (end 132.08 83.058) (width 0.3) (layer "F.Cu") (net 21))
 (segment (start 137.08 88.138) (end 132.08 88.138) (width 0.3) (layer "F.Cu") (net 23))
 (segment (start 132.08 75.438) (end 137.08 75.438) (width 0.3) (layer "F.Cu") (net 18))
 (segment (start 137.08 77.978) (end 132.08 77.978) (width 0.3) (layer "F.Cu") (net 19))
 (segment (start 165.02 85.598) (end 170.02 85.598) (width 0.3) (layer "F.Cu") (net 37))
 (segment (start 178.326 50.616) (end 173.138 50.616) (width 0.3) (layer "F.Cu") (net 25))
 (segment (start 179.526 51.816) (end 178.326 50.616) (width 0.3) (layer "F.Cu") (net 25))
 (segment (start 173.138 50.616) (end 170.02 47.498) (width 0.3) (layer "F.Cu") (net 25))
 (segment (start 170.02 47.498) (end 165.02 47.498) (width 0.3) (layer "F.Cu") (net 25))
 (segment (start 195.58 51.816) (end 179.526 51.816) (width 0.3) (layer "B.Cu") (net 25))
 (segment (start 208.923625 65.159625) (end 195.58 51.816) (width 0.3) (layer "B.Cu") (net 25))
 (segment (start 208.923625 69.0905) (end 208.923625 65.159625) (width 0.3) (layer "B.Cu") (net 25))
 (segment (start 170.02 72.898) (end 165.02 72.898) (width 0.3) (layer "F.Cu") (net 32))
 (segment (start 176.986 49.989057) (end 170.517057 56.458) (width 0.3) (layer "B.Cu") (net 32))
 (segment (start 176.986 49.276) (end 176.986 49.989057) (width 0.3) (layer "B.Cu") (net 32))
 (segment (start 168.82 57.160943) (end 168.82 71.698) (width 0.3) (layer "B.Cu") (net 32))
 (segment (start 170.517057 56.458) (end 169.522943 56.458) (width 0.3) (layer "B.Cu") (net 32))
 (segment (start 168.82 71.698) (end 170.02 72.898) (width 0.3) (layer "B.Cu") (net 32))
 (segment (start 169.522943 56.458) (end 168.82 57.160943) (width 0.3) (layer "B.Cu") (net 32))
 (segment (start 165.02 60.198) (end 170.02 60.198) (width 0.3) (layer "F.Cu") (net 28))
 (segment (start 170.02 52.578) (end 165.02 52.578) (width 0.3) (layer "F.Cu") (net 26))
 (segment (start 170.02 88.138) (end 165.02 88.138) (width 0.3) (layer "F.Cu") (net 38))
 (segment (start 188.923625 69.0905) (end 185.111125 65.278) (width 0.3) (layer "F.Cu") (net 30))
 (segment (start 185.111125 65.278) (end 170.02 65.278) (width 0.3) (layer "F.Cu") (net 30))
 (segment (start 165.02 65.278) (end 170.02 65.278) (width 0.3) (layer "F.Cu") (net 30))
 (segment (start 176.986 51.816) (end 171.22 57.582) (width 0.3) (layer "B.Cu") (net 30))
 (segment (start 171.22 64.078) (end 170.02 65.278) (width 0.3) (layer "B.Cu") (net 30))
 (segment (start 171.22 57.582) (end 171.22 64.078) (width 0.3) (layer "B.Cu") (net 30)))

